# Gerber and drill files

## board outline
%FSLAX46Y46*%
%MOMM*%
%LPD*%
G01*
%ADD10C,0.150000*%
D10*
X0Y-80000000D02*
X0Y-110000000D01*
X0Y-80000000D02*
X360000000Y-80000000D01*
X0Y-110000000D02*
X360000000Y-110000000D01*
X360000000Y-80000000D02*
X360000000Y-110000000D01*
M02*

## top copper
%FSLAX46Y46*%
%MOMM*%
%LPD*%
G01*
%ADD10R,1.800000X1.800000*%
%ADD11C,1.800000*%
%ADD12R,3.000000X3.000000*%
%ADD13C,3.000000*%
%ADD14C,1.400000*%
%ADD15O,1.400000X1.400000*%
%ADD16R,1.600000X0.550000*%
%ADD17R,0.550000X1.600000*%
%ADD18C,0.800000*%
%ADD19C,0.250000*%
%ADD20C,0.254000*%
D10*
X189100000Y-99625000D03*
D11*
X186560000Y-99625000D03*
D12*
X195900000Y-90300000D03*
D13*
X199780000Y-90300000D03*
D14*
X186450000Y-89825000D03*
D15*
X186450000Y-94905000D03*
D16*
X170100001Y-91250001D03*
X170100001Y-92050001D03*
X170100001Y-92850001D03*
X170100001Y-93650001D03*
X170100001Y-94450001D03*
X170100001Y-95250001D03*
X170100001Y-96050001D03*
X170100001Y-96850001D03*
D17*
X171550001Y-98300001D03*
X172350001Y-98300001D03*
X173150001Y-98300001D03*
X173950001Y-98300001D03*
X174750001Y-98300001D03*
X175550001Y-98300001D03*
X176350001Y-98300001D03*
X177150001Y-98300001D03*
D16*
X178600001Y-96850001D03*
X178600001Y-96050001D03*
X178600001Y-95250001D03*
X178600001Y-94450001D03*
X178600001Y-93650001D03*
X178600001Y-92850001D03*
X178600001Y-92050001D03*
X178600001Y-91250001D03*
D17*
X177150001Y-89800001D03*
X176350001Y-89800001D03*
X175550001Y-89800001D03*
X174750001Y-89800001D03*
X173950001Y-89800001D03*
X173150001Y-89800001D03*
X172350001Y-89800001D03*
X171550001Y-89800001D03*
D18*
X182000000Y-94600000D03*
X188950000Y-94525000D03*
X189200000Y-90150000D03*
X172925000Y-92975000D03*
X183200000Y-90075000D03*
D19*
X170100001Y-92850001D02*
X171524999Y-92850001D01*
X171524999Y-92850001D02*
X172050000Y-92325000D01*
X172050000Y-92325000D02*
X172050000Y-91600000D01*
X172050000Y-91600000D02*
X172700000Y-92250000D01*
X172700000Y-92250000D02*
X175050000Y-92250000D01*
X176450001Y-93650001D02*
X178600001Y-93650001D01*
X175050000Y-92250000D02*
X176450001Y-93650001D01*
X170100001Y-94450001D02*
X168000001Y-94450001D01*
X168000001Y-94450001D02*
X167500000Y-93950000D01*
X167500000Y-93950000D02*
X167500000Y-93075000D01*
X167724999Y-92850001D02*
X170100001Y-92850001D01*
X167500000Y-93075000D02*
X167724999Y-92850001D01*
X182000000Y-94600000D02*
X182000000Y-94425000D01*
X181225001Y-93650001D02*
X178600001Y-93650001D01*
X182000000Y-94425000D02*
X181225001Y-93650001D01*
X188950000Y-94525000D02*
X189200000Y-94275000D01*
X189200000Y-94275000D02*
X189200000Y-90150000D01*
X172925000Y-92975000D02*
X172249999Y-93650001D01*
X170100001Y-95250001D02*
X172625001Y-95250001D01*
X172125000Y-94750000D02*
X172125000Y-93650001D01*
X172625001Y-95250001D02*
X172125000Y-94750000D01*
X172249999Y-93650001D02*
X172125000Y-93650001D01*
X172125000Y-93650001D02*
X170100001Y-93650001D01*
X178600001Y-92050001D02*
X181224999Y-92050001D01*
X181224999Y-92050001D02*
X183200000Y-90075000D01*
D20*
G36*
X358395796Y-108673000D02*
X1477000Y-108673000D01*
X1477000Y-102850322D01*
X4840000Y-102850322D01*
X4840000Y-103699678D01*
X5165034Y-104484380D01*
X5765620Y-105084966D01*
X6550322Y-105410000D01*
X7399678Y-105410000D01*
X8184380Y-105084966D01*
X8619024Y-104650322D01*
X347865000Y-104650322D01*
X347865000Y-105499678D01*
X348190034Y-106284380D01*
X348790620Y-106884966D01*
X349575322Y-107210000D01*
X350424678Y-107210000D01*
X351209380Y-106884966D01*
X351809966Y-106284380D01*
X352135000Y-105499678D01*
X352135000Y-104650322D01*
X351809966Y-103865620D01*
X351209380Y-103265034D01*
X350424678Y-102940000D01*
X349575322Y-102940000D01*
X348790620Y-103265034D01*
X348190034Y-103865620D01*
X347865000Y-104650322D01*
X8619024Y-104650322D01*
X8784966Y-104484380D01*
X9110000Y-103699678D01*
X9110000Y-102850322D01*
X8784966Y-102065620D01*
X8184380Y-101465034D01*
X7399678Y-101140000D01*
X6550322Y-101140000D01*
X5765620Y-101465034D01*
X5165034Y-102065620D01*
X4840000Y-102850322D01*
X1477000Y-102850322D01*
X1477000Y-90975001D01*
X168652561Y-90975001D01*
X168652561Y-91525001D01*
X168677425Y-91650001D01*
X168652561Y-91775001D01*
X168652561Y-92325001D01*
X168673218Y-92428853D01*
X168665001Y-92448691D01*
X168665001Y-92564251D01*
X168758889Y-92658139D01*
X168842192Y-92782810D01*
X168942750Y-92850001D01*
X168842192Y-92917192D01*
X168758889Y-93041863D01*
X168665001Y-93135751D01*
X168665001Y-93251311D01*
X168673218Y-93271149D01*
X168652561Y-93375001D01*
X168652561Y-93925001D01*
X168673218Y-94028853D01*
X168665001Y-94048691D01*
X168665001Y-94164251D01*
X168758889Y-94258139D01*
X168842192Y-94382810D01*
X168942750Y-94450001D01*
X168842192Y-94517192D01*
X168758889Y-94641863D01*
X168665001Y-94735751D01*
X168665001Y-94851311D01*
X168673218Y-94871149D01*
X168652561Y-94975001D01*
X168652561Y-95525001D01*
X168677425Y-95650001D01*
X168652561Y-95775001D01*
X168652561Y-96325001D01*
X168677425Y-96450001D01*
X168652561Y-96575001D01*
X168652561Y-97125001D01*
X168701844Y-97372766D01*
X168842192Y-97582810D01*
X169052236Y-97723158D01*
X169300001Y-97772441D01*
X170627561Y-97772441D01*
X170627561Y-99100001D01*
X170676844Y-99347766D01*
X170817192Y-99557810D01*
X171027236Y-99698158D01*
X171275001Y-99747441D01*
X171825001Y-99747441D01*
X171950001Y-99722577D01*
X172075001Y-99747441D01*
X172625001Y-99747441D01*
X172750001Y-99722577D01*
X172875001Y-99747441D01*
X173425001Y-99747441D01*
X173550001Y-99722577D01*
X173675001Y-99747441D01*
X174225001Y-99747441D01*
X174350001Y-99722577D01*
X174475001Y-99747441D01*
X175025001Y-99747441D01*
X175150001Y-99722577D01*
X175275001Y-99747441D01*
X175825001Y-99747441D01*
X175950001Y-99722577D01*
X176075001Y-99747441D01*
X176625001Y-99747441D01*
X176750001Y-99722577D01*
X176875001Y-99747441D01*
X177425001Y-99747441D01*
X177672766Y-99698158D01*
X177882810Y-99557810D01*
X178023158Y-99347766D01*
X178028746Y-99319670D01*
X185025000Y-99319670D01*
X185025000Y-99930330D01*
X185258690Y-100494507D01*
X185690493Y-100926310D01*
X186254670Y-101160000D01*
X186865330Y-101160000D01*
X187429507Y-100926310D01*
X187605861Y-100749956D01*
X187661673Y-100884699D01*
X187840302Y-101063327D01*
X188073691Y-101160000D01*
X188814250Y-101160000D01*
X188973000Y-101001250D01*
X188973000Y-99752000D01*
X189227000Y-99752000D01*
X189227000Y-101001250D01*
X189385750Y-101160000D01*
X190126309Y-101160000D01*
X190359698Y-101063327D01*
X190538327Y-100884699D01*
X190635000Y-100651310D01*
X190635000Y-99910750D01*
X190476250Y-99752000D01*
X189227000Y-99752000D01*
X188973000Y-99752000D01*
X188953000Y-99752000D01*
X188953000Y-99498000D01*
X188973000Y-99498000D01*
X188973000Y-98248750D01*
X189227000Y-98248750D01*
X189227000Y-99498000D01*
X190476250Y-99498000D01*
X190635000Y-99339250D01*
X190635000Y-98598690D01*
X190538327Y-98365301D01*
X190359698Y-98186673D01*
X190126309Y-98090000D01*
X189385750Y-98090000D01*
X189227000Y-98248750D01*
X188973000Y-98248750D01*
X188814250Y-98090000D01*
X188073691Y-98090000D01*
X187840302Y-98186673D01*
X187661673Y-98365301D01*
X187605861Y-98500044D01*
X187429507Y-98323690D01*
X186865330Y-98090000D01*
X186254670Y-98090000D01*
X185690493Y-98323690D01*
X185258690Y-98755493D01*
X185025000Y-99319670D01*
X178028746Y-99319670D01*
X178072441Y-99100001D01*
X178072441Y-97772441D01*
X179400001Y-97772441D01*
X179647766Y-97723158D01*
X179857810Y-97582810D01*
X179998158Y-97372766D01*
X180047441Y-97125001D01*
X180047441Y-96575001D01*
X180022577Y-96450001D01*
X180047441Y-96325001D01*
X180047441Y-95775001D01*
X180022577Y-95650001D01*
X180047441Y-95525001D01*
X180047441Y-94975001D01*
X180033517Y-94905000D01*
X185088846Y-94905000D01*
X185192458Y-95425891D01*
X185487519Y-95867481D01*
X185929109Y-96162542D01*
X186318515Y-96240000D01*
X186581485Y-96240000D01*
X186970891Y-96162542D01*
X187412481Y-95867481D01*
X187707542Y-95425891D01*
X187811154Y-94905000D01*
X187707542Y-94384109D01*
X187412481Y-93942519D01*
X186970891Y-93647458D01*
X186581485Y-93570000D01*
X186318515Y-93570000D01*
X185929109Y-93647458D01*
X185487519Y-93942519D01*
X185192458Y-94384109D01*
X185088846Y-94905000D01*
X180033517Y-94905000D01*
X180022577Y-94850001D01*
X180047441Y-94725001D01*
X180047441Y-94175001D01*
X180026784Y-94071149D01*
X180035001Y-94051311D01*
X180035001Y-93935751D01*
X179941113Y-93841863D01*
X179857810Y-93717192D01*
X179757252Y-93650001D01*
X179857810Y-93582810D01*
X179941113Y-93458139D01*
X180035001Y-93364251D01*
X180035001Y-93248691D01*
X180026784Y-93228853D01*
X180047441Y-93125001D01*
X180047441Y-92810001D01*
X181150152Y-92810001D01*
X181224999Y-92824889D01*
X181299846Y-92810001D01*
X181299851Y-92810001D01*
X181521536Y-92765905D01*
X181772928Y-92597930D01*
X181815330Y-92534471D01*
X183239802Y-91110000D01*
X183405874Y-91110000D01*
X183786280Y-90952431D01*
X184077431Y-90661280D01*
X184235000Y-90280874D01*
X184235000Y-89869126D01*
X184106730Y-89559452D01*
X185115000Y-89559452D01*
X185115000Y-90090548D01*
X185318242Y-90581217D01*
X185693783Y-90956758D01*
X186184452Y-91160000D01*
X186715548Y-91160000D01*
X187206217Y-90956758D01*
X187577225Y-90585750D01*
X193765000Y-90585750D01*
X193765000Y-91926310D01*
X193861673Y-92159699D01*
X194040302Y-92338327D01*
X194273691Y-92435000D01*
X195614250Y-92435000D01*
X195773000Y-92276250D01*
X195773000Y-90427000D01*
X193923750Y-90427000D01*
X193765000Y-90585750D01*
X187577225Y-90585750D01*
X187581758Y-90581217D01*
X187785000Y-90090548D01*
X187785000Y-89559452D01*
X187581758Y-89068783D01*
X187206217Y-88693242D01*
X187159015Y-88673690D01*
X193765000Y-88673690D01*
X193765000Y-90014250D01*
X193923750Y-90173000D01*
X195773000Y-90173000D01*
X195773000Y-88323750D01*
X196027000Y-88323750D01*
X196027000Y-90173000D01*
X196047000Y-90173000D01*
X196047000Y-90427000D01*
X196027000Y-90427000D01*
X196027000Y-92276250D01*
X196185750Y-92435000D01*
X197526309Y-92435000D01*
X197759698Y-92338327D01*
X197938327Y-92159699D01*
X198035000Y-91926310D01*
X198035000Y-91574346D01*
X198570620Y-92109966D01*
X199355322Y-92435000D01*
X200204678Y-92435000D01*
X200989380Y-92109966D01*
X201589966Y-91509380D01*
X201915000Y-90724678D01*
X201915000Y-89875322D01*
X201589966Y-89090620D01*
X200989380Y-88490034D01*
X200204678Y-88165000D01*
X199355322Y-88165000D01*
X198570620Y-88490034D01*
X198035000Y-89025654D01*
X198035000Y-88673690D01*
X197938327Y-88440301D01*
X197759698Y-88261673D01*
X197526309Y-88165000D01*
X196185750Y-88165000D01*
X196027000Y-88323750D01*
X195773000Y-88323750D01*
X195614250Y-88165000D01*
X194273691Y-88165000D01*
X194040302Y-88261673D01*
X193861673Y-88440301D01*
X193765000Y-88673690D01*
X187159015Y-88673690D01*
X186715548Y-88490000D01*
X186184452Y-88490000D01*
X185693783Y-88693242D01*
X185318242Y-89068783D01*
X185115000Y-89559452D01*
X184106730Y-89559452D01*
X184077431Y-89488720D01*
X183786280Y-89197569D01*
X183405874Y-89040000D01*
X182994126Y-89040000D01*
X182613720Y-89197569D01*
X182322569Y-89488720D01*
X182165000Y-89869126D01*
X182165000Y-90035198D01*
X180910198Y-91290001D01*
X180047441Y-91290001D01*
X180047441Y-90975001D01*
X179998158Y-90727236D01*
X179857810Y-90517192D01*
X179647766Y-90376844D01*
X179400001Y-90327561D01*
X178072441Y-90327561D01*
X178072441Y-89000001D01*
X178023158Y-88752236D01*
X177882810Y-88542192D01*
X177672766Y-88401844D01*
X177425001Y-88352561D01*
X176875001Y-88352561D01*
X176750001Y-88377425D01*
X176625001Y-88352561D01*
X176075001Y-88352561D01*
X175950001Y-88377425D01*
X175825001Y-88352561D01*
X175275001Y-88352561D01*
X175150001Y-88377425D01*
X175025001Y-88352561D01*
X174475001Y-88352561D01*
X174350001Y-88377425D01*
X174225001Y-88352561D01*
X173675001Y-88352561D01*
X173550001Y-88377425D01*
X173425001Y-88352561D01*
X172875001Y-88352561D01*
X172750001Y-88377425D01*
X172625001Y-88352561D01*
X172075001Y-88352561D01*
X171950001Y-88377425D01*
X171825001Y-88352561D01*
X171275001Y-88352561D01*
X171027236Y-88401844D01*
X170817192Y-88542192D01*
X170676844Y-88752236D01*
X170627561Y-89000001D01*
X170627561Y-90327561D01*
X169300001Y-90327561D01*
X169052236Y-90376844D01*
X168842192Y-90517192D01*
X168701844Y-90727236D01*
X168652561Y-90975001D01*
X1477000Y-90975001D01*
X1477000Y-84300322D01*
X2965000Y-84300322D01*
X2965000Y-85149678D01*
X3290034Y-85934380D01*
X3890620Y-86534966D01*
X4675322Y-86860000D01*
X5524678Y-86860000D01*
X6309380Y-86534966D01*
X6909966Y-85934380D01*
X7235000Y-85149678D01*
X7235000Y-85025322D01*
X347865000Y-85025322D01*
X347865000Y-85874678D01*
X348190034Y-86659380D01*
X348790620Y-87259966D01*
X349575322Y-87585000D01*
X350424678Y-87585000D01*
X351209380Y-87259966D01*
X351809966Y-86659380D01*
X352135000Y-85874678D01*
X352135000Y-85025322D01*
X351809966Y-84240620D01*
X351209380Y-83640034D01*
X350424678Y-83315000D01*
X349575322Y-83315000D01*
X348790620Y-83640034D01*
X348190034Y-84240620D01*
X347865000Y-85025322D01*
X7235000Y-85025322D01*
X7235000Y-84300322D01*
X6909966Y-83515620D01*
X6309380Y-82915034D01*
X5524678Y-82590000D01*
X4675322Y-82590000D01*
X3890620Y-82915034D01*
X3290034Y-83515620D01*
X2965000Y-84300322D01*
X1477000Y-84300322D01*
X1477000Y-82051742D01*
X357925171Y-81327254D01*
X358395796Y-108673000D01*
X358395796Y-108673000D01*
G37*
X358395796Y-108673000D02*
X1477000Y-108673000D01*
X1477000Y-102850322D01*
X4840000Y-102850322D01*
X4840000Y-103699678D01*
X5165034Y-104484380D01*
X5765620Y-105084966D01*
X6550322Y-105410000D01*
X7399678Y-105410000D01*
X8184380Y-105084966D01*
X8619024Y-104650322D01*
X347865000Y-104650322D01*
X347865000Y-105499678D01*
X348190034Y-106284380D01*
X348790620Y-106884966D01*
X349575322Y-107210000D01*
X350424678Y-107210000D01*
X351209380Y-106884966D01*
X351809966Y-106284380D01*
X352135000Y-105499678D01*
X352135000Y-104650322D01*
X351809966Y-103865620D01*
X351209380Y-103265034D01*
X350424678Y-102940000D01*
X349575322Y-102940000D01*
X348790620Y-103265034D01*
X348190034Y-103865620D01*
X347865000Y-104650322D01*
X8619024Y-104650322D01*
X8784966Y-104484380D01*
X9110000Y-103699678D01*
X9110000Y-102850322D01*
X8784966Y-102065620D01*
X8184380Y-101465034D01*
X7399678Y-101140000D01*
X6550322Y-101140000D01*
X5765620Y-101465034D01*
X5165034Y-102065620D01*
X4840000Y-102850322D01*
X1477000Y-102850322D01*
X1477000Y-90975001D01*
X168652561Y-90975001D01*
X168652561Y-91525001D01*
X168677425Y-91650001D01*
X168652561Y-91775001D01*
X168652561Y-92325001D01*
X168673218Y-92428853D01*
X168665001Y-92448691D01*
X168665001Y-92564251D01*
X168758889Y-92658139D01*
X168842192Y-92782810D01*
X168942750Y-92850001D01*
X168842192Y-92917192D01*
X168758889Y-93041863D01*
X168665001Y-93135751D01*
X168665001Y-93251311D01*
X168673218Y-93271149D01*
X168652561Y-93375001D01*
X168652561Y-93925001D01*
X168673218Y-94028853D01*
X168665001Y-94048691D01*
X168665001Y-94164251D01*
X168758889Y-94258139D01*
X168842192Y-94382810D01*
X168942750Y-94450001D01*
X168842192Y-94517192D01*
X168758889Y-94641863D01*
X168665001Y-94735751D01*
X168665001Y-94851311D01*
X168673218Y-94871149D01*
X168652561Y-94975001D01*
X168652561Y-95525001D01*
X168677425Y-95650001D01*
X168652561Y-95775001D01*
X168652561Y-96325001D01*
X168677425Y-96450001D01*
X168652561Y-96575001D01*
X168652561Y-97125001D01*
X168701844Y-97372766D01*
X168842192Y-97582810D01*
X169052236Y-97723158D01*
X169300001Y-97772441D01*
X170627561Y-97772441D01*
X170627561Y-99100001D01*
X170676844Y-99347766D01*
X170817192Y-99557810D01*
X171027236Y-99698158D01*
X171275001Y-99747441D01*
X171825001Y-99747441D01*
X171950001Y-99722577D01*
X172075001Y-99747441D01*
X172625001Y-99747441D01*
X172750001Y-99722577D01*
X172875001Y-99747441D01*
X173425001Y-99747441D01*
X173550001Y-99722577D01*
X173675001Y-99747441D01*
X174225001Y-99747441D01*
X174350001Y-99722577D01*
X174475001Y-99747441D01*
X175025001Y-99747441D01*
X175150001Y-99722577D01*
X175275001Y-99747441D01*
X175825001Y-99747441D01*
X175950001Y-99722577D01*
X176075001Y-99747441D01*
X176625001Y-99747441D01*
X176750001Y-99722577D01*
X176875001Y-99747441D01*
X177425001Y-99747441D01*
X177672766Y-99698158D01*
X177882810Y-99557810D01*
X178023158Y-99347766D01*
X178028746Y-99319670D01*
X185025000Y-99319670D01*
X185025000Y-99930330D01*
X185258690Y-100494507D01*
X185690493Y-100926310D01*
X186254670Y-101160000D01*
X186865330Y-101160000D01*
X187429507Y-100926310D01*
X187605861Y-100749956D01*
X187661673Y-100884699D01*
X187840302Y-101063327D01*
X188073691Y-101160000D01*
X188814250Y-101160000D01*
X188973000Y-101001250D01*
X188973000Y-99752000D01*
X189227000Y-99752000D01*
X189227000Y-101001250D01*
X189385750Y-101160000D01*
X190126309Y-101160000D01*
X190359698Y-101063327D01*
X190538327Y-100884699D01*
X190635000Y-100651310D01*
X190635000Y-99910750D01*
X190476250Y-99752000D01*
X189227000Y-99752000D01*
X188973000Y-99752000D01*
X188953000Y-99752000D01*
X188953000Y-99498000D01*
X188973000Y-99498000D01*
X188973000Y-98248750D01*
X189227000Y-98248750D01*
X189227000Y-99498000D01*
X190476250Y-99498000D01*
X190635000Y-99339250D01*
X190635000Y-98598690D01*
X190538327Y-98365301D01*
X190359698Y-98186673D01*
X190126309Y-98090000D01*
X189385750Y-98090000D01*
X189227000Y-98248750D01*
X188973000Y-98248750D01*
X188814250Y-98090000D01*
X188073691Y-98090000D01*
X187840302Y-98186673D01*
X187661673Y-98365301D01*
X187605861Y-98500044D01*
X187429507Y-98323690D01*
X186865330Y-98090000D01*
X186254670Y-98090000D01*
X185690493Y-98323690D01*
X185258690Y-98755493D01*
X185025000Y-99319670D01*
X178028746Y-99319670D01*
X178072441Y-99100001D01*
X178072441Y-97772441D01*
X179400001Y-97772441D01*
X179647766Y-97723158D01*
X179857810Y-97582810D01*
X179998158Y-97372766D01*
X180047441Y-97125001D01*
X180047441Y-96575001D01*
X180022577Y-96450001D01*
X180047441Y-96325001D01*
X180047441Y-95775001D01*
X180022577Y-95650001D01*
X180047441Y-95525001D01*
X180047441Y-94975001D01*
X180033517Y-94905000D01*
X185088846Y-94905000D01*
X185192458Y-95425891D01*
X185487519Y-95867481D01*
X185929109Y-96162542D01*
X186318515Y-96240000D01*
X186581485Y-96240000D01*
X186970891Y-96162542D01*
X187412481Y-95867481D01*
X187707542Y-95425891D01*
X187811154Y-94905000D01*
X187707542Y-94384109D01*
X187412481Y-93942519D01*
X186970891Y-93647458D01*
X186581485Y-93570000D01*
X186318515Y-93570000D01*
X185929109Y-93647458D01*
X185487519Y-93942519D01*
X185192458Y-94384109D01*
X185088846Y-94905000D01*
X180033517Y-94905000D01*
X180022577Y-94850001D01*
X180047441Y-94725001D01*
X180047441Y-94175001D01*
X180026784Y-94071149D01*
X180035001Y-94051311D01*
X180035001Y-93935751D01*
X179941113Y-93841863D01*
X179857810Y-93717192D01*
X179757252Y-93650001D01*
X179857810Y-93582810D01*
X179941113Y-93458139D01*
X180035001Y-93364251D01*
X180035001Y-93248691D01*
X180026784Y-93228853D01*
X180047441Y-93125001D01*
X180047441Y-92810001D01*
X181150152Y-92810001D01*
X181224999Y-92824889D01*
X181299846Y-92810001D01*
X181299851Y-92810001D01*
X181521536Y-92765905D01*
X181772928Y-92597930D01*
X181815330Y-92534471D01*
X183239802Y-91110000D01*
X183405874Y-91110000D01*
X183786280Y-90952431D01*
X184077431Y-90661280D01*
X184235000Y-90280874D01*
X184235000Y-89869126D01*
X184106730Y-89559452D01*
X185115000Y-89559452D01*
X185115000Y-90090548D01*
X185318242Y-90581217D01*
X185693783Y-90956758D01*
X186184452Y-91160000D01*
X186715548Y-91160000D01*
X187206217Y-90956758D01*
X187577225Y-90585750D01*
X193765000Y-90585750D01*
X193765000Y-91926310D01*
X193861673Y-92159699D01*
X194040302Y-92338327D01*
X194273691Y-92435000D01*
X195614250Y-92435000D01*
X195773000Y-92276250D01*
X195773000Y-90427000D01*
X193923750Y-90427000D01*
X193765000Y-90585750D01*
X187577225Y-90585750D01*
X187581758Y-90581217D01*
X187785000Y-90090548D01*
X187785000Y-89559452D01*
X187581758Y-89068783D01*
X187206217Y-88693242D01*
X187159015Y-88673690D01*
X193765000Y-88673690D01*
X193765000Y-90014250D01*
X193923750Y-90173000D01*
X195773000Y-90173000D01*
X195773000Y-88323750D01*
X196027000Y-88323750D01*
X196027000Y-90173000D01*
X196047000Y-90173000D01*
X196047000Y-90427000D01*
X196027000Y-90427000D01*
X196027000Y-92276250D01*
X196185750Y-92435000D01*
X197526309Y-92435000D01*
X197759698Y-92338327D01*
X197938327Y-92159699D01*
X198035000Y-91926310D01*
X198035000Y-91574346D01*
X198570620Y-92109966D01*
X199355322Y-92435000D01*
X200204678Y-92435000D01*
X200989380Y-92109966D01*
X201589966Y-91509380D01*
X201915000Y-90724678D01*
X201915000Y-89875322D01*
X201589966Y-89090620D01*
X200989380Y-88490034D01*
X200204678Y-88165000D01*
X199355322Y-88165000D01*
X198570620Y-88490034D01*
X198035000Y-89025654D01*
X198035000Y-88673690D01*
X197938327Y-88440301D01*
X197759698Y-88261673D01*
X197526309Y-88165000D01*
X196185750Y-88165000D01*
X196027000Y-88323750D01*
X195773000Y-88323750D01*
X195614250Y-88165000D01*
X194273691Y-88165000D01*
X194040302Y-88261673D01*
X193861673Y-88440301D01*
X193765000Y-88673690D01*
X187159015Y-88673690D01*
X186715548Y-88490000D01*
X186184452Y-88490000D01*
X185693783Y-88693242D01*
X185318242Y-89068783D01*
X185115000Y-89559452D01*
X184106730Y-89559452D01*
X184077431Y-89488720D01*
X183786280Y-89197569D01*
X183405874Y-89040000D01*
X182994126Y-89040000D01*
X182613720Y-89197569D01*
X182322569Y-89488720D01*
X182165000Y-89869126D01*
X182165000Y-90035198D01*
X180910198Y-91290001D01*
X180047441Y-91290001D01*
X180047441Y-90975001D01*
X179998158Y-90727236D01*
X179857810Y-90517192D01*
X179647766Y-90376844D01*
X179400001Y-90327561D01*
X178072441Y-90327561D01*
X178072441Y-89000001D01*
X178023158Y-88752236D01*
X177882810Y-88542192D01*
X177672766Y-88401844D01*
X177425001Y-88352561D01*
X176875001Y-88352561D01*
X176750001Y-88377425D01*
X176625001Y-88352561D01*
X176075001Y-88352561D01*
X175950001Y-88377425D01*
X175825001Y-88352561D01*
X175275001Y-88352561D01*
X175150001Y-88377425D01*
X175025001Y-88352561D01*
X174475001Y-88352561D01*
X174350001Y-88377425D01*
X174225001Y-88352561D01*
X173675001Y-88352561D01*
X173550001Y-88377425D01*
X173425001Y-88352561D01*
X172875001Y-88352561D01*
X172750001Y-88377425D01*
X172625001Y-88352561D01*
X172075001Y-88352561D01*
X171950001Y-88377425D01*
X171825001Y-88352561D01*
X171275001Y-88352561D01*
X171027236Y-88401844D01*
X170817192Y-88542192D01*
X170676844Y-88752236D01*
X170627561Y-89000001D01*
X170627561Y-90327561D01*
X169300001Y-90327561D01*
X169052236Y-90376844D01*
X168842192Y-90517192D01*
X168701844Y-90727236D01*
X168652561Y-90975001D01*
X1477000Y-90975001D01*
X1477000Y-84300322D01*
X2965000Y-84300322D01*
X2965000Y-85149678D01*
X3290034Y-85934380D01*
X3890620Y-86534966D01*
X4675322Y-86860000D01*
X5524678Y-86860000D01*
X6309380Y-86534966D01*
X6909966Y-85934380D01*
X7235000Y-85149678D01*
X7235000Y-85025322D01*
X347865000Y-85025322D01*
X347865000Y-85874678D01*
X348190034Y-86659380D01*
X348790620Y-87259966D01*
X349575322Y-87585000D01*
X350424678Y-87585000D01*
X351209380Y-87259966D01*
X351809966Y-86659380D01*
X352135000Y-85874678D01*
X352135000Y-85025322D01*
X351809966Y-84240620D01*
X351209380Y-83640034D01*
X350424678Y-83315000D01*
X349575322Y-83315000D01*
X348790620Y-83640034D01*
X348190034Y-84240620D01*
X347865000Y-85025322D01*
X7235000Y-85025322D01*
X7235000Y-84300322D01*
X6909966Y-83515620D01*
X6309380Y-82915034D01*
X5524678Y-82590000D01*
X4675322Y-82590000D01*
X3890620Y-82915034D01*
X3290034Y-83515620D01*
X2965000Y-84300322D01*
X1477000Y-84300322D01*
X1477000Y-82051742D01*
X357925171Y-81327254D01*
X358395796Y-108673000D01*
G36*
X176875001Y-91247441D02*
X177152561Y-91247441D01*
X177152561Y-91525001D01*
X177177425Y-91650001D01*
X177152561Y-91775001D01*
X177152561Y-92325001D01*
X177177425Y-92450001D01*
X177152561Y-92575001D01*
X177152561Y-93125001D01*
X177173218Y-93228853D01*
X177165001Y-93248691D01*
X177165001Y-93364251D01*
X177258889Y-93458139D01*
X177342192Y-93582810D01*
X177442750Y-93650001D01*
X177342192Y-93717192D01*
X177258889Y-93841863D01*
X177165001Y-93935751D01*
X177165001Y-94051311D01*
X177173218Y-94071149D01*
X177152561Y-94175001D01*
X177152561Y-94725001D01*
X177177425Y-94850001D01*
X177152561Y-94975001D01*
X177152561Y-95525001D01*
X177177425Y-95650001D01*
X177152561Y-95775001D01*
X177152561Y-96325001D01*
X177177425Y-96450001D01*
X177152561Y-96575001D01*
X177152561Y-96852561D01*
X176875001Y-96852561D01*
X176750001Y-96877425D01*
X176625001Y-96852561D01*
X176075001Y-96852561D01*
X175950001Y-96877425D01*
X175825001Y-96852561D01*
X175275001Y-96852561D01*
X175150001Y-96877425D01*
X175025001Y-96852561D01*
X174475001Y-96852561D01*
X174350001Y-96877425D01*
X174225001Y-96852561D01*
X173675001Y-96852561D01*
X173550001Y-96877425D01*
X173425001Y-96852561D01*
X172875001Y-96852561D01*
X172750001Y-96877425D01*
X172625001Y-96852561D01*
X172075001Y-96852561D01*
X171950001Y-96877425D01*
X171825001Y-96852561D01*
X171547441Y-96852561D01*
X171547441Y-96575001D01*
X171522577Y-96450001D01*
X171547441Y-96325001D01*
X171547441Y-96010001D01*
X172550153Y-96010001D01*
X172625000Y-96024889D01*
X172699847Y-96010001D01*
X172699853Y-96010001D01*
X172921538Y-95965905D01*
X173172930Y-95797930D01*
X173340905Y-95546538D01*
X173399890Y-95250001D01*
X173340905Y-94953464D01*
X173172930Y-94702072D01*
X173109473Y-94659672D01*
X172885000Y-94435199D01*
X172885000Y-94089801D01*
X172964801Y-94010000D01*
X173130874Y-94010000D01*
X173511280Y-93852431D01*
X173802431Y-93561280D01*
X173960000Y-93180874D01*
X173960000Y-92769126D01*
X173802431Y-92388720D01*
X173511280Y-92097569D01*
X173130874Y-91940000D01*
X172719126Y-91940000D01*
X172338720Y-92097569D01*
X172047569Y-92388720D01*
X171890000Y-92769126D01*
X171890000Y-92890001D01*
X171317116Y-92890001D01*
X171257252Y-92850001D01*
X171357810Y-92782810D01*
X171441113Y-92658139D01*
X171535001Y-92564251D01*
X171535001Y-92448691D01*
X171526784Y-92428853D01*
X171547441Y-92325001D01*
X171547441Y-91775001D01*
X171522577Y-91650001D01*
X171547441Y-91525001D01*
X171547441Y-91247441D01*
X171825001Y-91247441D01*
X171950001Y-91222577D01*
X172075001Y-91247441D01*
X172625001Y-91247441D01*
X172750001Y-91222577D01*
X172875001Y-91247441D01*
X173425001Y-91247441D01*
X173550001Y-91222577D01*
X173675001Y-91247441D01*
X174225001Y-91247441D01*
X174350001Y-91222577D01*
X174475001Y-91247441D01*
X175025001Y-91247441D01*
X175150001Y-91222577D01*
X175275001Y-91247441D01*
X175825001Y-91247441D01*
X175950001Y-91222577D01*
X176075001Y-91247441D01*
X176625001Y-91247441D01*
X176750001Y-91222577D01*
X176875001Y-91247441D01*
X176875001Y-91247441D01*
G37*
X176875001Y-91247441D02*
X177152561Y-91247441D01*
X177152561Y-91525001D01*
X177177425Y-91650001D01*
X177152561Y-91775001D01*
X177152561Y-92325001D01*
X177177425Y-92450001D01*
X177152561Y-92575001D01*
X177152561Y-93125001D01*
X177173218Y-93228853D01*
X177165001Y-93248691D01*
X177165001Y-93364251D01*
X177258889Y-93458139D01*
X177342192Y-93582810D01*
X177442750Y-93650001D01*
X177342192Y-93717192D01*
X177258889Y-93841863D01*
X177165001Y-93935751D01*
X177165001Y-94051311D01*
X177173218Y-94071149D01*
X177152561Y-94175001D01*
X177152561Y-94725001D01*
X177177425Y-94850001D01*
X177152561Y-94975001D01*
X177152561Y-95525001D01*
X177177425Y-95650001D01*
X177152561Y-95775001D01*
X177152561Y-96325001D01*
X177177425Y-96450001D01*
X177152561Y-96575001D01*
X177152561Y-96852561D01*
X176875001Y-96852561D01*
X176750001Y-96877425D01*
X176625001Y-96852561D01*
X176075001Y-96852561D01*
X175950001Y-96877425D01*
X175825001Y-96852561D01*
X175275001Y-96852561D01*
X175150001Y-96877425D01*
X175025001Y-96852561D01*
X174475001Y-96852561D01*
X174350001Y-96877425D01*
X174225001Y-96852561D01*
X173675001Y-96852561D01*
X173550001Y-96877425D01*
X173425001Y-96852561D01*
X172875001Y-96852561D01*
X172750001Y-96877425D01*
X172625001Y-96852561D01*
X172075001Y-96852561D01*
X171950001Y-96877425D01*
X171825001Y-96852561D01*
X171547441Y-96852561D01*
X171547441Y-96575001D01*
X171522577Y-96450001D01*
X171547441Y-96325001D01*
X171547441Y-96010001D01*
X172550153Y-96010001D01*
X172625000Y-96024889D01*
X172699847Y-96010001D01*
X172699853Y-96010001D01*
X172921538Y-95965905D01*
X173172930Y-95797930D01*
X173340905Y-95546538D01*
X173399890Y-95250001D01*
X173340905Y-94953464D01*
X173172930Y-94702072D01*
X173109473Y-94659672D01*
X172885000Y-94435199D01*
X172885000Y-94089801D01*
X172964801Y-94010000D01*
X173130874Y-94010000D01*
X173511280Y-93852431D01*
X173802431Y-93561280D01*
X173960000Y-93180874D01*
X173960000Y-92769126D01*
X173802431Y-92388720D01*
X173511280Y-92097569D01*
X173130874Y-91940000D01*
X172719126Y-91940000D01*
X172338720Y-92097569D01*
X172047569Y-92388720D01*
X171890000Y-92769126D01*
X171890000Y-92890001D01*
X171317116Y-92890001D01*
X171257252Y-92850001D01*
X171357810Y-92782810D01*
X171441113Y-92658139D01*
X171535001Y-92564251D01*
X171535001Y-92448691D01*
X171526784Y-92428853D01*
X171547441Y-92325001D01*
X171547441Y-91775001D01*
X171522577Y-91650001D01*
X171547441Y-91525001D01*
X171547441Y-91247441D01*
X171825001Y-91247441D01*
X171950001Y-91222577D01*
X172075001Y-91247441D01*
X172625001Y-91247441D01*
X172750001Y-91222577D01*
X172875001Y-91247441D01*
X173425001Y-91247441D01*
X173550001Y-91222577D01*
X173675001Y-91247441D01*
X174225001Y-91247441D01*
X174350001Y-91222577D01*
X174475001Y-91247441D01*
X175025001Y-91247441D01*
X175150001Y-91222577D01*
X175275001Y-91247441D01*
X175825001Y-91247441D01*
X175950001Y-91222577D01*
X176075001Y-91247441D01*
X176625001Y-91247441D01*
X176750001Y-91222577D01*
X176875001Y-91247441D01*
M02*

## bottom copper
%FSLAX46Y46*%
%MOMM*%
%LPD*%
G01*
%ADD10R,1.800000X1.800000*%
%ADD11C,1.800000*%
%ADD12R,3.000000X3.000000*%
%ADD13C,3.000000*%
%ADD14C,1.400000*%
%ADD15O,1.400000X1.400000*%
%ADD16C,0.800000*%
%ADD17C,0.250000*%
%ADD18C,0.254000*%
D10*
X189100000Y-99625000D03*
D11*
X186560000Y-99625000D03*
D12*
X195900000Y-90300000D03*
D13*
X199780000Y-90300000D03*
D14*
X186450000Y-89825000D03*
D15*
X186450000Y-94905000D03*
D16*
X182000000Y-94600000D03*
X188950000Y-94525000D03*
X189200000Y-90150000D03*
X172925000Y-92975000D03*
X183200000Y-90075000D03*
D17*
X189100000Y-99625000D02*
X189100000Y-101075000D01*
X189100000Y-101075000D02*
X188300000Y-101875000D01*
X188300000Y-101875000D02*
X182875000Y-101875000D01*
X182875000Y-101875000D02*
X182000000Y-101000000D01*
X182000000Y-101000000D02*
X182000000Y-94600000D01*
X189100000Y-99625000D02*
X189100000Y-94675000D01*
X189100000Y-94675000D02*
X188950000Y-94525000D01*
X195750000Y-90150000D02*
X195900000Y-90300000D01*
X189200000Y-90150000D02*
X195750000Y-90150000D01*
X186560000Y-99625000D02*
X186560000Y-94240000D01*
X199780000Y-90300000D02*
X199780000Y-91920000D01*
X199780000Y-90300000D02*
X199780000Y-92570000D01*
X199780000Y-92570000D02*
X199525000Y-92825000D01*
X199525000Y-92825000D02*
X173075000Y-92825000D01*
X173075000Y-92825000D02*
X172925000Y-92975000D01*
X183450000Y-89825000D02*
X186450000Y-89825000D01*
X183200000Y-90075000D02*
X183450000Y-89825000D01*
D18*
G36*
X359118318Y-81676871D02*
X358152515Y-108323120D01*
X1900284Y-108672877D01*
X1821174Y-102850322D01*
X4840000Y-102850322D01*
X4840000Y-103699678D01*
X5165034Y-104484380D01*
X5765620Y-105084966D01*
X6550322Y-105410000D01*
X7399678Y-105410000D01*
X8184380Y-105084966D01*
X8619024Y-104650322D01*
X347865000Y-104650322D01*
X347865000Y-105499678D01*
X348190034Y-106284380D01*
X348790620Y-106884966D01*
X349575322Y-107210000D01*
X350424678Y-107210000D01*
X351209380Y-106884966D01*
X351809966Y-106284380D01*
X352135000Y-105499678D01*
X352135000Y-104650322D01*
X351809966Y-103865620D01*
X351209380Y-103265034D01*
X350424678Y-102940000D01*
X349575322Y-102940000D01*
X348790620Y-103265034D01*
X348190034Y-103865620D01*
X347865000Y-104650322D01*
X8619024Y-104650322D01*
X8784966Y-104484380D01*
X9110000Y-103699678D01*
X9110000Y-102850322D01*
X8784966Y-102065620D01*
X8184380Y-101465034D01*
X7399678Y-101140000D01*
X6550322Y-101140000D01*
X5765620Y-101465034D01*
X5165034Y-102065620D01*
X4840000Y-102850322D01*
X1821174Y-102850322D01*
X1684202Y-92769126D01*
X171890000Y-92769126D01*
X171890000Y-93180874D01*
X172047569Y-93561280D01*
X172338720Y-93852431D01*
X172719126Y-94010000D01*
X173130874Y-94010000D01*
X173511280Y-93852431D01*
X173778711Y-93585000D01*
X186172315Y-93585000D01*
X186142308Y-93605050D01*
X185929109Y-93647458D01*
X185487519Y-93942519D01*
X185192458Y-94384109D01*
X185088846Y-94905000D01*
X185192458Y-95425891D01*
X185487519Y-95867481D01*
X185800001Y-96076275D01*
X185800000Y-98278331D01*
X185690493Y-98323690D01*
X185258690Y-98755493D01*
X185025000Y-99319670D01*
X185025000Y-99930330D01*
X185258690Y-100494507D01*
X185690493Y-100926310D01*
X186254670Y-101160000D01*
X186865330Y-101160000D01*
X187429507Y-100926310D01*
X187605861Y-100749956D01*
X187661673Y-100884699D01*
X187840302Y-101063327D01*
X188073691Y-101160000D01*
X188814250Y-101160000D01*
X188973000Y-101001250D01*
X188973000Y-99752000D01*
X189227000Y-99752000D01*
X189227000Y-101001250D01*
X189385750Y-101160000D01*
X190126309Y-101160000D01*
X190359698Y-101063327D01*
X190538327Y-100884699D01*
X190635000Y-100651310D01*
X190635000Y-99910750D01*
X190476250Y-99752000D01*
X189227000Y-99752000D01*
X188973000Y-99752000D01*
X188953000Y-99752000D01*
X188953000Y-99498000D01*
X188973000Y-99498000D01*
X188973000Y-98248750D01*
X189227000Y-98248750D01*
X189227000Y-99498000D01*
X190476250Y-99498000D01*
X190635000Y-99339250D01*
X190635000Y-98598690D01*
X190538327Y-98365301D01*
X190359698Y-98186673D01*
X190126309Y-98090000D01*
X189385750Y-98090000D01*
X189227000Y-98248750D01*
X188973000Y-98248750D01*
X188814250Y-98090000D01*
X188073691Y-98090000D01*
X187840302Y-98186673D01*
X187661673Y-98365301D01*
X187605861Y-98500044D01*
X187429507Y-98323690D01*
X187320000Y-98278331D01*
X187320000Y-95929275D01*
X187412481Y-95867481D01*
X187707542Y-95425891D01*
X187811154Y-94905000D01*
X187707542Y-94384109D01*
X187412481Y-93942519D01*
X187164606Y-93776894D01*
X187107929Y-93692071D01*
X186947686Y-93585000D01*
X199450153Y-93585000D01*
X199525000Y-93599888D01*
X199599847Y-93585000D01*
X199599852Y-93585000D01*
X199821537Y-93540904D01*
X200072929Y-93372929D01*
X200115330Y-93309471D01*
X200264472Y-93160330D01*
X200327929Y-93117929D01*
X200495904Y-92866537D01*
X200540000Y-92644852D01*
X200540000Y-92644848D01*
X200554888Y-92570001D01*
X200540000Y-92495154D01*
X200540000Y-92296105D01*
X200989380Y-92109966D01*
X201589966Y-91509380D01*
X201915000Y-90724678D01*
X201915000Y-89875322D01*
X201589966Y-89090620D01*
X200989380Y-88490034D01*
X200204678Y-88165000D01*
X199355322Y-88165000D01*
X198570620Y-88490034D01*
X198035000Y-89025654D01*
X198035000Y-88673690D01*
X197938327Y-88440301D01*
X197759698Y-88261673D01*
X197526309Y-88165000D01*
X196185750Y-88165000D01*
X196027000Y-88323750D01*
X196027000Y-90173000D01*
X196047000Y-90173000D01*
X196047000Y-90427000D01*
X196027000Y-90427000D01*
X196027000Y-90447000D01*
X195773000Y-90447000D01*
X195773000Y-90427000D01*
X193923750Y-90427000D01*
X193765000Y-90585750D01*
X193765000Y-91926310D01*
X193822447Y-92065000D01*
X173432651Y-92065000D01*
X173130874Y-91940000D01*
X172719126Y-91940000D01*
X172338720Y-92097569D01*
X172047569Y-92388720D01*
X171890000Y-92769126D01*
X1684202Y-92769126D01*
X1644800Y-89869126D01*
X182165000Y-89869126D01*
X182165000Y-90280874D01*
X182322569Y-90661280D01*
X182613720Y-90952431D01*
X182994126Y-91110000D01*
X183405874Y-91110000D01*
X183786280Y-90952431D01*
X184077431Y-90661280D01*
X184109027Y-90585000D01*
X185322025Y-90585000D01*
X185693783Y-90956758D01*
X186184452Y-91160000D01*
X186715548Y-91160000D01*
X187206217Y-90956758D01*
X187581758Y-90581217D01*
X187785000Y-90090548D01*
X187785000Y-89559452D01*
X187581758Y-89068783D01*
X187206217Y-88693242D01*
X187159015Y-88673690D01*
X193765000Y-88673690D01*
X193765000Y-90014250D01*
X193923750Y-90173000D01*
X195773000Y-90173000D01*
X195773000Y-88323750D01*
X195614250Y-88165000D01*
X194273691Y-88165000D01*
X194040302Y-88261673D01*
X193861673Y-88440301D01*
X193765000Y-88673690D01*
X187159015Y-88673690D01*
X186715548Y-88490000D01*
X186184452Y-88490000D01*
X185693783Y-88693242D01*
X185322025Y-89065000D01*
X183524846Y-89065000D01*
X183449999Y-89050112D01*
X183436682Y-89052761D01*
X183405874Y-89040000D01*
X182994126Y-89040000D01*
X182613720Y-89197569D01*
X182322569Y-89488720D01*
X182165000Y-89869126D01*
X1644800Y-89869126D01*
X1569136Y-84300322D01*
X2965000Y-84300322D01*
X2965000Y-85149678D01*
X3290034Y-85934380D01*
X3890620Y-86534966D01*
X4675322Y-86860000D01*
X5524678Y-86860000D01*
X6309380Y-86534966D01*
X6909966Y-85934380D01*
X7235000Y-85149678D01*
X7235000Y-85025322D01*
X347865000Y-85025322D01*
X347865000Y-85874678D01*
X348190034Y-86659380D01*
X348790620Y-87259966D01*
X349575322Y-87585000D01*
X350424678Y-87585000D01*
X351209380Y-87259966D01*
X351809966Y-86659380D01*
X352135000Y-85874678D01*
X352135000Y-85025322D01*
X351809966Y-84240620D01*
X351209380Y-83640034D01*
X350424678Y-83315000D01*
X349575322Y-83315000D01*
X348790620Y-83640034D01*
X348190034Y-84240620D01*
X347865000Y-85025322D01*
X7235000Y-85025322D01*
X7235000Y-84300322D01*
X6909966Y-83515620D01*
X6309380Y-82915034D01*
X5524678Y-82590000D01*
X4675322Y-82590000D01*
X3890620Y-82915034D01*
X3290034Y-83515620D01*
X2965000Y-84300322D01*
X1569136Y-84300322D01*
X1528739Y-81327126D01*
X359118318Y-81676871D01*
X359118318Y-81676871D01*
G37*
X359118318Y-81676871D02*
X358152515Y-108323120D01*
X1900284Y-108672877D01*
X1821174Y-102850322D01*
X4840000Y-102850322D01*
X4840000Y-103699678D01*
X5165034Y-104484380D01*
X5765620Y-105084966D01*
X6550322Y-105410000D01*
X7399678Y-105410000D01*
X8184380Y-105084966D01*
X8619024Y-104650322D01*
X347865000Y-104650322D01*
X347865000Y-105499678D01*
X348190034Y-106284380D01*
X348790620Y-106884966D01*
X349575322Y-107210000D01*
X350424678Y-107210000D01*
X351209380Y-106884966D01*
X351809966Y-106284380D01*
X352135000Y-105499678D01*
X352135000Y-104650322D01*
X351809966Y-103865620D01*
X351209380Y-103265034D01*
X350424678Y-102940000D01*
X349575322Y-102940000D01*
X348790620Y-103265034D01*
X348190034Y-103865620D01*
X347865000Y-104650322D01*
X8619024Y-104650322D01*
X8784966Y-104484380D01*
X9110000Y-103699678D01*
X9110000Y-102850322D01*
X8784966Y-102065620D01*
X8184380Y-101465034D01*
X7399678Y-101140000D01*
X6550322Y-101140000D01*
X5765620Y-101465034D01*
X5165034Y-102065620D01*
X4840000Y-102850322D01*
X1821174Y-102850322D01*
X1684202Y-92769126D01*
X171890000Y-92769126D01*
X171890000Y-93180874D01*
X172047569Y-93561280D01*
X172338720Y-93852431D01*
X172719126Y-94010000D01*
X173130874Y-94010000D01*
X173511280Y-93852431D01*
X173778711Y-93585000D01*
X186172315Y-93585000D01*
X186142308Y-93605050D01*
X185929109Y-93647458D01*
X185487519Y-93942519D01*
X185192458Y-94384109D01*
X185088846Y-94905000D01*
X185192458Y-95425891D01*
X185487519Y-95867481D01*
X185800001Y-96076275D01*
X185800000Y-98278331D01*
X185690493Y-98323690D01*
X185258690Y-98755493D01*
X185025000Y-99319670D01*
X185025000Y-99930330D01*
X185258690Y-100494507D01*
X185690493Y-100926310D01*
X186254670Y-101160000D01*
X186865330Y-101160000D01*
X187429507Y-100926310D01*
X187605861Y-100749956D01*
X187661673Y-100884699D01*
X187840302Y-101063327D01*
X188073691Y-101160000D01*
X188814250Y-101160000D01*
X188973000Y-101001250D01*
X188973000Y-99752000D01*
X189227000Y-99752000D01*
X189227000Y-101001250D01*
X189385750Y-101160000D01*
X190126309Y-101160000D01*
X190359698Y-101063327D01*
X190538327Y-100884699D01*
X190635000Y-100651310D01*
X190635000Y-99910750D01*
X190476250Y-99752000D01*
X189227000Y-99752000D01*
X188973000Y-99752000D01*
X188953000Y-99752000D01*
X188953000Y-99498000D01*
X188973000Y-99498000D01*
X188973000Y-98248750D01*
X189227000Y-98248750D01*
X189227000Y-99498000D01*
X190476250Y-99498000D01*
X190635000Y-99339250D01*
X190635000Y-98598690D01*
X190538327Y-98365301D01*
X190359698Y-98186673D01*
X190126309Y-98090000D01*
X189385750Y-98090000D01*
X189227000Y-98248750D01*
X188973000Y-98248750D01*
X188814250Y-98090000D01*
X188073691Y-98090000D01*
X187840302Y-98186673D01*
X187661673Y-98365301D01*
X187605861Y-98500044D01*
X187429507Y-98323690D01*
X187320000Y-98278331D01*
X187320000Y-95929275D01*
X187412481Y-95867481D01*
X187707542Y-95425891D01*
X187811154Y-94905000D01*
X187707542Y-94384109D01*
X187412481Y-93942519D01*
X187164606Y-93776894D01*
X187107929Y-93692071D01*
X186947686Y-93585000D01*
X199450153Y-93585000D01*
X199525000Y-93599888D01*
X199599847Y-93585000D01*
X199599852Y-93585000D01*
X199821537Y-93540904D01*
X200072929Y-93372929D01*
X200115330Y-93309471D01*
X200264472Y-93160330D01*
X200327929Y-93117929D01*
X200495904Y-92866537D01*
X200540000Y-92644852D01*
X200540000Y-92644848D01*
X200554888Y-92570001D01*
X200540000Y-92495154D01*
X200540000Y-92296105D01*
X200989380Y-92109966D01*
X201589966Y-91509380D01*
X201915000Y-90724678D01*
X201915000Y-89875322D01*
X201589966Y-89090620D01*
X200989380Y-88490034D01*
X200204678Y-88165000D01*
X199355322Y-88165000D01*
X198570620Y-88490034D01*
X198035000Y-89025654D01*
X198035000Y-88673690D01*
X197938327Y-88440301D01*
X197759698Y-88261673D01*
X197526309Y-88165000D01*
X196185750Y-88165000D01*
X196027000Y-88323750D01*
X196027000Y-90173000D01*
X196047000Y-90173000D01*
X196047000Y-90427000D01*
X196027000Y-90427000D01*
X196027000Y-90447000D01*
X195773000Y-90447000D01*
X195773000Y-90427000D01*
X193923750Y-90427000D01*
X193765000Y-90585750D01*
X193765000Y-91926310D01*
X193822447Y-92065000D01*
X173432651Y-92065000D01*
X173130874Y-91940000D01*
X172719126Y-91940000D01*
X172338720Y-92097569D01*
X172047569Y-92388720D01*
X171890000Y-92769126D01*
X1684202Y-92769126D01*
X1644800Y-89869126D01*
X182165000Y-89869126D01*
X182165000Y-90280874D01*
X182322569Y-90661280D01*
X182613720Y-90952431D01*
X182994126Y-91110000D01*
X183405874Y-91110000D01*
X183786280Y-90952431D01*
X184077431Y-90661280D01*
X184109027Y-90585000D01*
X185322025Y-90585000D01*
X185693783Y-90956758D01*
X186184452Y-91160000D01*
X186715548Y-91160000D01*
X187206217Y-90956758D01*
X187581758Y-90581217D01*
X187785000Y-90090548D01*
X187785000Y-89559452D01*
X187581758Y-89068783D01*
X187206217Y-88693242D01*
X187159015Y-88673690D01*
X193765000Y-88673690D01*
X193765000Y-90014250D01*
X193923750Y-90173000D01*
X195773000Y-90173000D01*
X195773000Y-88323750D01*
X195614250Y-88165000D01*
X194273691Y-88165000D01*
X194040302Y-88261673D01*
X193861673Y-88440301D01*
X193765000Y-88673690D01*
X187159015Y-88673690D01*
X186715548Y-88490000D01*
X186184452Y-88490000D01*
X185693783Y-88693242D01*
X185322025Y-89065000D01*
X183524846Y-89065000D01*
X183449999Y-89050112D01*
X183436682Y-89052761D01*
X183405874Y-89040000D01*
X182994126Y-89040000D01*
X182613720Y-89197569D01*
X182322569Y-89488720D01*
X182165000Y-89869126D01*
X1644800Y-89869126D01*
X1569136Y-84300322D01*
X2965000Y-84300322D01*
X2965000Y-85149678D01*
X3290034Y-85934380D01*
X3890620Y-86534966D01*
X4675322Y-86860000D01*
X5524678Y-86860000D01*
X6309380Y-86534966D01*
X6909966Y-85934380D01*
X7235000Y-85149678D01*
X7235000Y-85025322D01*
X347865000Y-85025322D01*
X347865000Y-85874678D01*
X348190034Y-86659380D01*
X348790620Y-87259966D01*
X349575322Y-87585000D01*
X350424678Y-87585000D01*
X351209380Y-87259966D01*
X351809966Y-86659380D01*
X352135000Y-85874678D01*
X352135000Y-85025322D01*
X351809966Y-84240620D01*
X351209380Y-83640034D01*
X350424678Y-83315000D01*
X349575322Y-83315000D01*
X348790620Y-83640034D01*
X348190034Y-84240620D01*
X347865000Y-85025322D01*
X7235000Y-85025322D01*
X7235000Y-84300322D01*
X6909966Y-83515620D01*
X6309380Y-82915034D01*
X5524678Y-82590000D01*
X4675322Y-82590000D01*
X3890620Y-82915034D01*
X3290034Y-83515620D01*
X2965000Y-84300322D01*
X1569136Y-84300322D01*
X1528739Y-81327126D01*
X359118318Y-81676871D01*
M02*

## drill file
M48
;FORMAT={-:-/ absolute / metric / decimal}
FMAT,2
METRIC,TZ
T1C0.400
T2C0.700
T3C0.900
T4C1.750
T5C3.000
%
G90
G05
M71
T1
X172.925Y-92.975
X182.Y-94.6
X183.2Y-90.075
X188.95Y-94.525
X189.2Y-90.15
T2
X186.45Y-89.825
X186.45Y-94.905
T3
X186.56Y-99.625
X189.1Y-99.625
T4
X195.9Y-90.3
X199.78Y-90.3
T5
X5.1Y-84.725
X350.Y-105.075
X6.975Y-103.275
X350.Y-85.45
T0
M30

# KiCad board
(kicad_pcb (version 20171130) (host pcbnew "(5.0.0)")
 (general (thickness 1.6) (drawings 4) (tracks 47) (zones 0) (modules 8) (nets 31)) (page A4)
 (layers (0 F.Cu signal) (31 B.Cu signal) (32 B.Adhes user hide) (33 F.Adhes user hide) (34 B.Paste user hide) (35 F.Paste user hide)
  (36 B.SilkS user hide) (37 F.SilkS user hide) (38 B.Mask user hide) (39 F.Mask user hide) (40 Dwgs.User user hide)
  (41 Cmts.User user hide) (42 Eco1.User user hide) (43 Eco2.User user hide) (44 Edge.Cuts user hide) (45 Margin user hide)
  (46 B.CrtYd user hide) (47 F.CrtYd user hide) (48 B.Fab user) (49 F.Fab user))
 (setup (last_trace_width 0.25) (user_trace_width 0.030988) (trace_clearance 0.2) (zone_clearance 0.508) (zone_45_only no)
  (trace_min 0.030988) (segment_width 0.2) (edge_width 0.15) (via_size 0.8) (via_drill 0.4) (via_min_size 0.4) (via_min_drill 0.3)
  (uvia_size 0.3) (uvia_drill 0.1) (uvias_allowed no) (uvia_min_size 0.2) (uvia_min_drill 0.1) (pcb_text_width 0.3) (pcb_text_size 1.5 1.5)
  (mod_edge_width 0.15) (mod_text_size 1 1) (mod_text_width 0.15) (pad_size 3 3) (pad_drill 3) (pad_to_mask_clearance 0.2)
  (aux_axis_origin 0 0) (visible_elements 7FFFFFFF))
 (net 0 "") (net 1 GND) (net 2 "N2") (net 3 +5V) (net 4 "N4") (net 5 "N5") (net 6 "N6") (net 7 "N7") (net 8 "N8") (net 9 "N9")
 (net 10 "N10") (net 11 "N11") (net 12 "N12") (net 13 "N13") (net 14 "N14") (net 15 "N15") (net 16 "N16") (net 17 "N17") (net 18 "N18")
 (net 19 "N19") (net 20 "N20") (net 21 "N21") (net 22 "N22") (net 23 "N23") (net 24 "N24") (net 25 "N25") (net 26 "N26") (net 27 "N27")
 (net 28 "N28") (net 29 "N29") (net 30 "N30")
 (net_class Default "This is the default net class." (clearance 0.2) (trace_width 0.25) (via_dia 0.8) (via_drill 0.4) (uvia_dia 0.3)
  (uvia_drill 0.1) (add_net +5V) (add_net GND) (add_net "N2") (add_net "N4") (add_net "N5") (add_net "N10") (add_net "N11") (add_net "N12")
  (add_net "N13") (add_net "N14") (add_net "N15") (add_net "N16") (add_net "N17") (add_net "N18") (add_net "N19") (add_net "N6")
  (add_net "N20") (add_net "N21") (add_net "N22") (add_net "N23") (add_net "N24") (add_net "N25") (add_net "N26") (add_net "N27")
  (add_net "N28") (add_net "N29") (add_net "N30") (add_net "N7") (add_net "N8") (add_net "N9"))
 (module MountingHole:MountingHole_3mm (layer F.Cu) (at 5.1 84.725)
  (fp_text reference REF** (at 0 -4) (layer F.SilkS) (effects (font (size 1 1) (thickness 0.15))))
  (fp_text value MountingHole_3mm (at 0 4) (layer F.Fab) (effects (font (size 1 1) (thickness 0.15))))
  (pad 1 np_thru_hole circle (at 0 0) (size 3 3) (drill 3) (layers *.Cu *.Mask)))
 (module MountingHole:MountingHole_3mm (layer F.Cu) (at 6.975 103.275)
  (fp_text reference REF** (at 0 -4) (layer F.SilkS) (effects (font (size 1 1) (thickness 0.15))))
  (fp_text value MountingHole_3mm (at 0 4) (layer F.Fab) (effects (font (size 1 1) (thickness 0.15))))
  (pad 1 np_thru_hole circle (at 0 0) (size 3 3) (drill 3) (layers *.Cu *.Mask)))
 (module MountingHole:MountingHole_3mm (layer F.Cu) (at 350 85.45 90)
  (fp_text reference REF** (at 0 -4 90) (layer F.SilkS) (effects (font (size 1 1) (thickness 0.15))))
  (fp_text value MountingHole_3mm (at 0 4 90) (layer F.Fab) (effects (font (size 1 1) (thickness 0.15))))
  (pad 1 np_thru_hole circle (at 0 0 90) (size 3 3) (drill 3) (layers *.Cu *.Mask)))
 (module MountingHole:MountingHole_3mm (layer F.Cu) (at 350 105.075)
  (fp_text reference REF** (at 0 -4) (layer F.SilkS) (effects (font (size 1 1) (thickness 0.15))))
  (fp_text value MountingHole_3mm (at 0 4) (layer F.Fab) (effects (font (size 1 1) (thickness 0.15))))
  (pad 1 np_thru_hole circle (at 0 0) (size 3 3) (drill 3) (layers *.Cu *.Mask)))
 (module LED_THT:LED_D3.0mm (layer F.Cu) (at 189.1 99.625 180)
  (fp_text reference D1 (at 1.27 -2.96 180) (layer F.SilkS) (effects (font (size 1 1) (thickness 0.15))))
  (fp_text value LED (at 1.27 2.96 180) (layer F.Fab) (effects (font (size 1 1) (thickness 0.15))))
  (pad 1 thru_hole rect (at 0 0 180) (size 1.8 1.8) (drill 0.9) (layers *.Cu *.Mask) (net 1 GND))
  (pad 2 thru_hole circle (at 2.54 0 180) (size 1.8 1.8) (drill 0.9) (layers *.Cu *.Mask) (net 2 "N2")))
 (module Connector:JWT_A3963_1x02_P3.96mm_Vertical (layer F.Cu) (at 195.9 90.3)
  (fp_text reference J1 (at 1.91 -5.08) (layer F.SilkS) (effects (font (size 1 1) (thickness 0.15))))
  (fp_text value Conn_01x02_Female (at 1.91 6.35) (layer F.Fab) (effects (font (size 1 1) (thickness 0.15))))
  (pad 1 thru_hole rect (at 0 0) (size 3 3) (drill 1.75) (layers *.Cu *.Mask) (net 1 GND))
  (pad 2 thru_hole circle (at 3.88 0) (size 3 3) (drill 1.75) (layers *.Cu *.Mask) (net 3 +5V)))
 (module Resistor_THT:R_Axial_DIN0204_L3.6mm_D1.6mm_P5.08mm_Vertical (layer F.Cu) (at 186.45 89.825 270)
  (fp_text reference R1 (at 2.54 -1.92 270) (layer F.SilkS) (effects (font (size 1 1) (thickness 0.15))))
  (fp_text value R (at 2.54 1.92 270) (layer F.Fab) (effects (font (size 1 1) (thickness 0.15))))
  (pad 1 thru_hole circle (at 0 0 270) (size 1.4 1.4) (drill 0.7) (layers *.Cu *.Mask) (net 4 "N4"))
  (pad 2 thru_hole oval (at 5.08 0 270) (size 1.4 1.4) (drill 0.7) (layers *.Cu *.Mask) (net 2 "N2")))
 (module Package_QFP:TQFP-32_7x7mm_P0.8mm (layer F.Cu) (at 174.350001 94.050001)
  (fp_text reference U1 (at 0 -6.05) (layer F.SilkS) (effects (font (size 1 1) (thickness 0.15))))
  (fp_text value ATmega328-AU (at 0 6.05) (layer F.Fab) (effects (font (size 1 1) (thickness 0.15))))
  (pad 1 smd rect (at -4.25 -2.8) (size 1.6 0.55) (layers F.Cu F.Paste F.Mask) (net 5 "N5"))
  (pad 2 smd rect (at -4.25 -2) (size 1.6 0.55) (layers F.Cu F.Paste F.Mask) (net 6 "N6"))
  (pad 3 smd rect (at -4.25 -1.2) (size 1.6 0.55) (layers F.Cu F.Paste F.Mask) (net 1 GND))
  (pad 4 smd rect (at -4.25 -0.4) (size 1.6 0.55) (layers F.Cu F.Paste F.Mask) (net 3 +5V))
  (pad 5 smd rect (at -4.25 0.4) (size 1.6 0.55) (layers F.Cu F.Paste F.Mask) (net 1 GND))
  (pad 6 smd rect (at -4.25 1.2) (size 1.6 0.55) (layers F.Cu F.Paste F.Mask) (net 3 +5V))
  (pad 7 smd rect (at -4.25 2) (size 1.6 0.55) (layers F.Cu F.Paste F.Mask) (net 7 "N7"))
  (pad 8 smd rect (at -4.25 2.8) (size 1.6 0.55) (layers F.Cu F.Paste F.Mask) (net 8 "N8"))
  (pad 9 smd rect (at -2.8 4.25 90) (size 1.6 0.55) (layers F.Cu F.Paste F.Mask) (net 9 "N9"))
  (pad 10 smd rect (at -2 4.25 90) (size 1.6 0.55) (layers F.Cu F.Paste F.Mask) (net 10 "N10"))
  (pad 11 smd rect (at -1.2 4.25 90) (size 1.6 0.55) (layers F.Cu F.Paste F.Mask) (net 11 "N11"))
  (pad 12 smd rect (at -0.4 4.25 90) (size 1.6 0.55) (layers F.Cu F.Paste F.Mask) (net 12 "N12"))
  (pad 13 smd rect (at 0.4 4.25 90) (size 1.6 0.55) (layers F.Cu F.Paste F.Mask) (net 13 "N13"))
  (pad 14 smd rect (at 1.2 4.25 90) (size 1.6 0.55) (layers F.Cu F.Paste F.Mask) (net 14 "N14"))
  (pad 15 smd rect (at 2 4.25 90) (size 1.6 0.55) (layers F.Cu F.Paste F.Mask) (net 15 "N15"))
  (pad 16 smd rect (at 2.8 4.25 90) (size 1.6 0.55) (layers F.Cu F.Paste F.Mask) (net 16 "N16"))
  (pad 17 smd rect (at 4.25 2.8) (size 1.6 0.55) (layers F.Cu F.Paste F.Mask) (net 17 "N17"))
  (pad 18 smd rect (at 4.25 2) (size 1.6 0.55) (layers F.Cu F.Paste F.Mask) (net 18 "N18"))
  (pad 19 smd rect (at 4.25 1.2) (size 1.6 0.55) (layers F.Cu F.Paste F.Mask) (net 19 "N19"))
  (pad 20 smd rect (at 4.25 0.4) (size 1.6 0.55) (layers F.Cu F.Paste F.Mask) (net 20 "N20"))
  (pad 21 smd rect (at 4.25 -0.4) (size 1.6 0.55) (layers F.Cu F.Paste F.Mask) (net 1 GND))
  (pad 22 smd rect (at 4.25 -1.2) (size 1.6 0.55) (layers F.Cu F.Paste F.Mask) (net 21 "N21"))
  (pad 23 smd rect (at 4.25 -2) (size 1.6 0.55) (layers F.Cu F.Paste F.Mask) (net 4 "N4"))
  (pad 24 smd rect (at 4.25 -2.8) (size 1.6 0.55) (layers F.Cu F.Paste F.Mask) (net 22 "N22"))
  (pad 25 smd rect (at 2.8 -4.25 90) (size 1.6 0.55) (layers F.Cu F.Paste F.Mask) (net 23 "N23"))
  (pad 26 smd rect (at 2 -4.25 90) (size 1.6 0.55) (layers F.Cu F.Paste F.Mask) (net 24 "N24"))
  (pad 27 smd rect (at 1.2 -4.25 90) (size 1.6 0.55) (layers F.Cu F.Paste F.Mask) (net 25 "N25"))
  (pad 28 smd rect (at 0.4 -4.25 90) (size 1.6 0.55) (layers F.Cu F.Paste F.Mask) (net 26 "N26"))
  (pad 29 smd rect (at -0.4 -4.25 90) (size 1.6 0.55) (layers F.Cu F.Paste F.Mask) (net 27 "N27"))
  (pad 30 smd rect (at -1.2 -4.25 90) (size 1.6 0.55) (layers F.Cu F.Paste F.Mask) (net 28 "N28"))
  (pad 31 smd rect (at -2 -4.25 90) (size 1.6 0.55) (layers F.Cu F.Paste F.Mask) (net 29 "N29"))
  (pad 32 smd rect (at -2.8 -4.25 90) (size 1.6 0.55) (layers F.Cu F.Paste F.Mask) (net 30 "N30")))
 (gr_line (start 0 80) (end 0 110) (layer Edge.Cuts) (width 0.15))
 (gr_line (start 0 80) (end 360 80) (layer Edge.Cuts) (width 0.15))
 (gr_line (start 0 110) (end 360 110) (layer Edge.Cuts) (width 0.15))
 (gr_line (start 360 80) (end 360 110) (layer Edge.Cuts) (width 0.15))
 (segment (start 170.100001 92.850001) (end 171.524999 92.850001) (width 0.25) (layer F.Cu) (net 1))
 (segment (start 171.524999 92.850001) (end 172.05 92.325) (width 0.25) (layer F.Cu) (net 1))
 (segment (start 172.05 92.325) (end 172.05 91.6) (width 0.25) (layer F.Cu) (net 1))
 (segment (start 172.05 91.6) (end 172.7 92.25) (width 0.25) (layer F.Cu) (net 1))
 (segment (start 172.7 92.25) (end 175.05 92.25) (width 0.25) (layer F.Cu) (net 1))
 (segment (start 176.450001 93.650001) (end 178.600001 93.650001) (width 0.25) (layer F.Cu) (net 1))
 (segment (start 175.05 92.25) (end 176.450001 93.650001) (width 0.25) (layer F.Cu) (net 1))
 (segment (start 170.100001 94.450001) (end 168.000001 94.450001) (width 0.25) (layer F.Cu) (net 1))
 (segment (start 168.000001 94.450001) (end 167.5 93.95) (width 0.25) (layer F.Cu) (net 1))
 (segment (start 167.5 93.95) (end 167.5 93.075) (width 0.25) (layer F.Cu) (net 1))
 (segment (start 167.724999 92.850001) (end 170.100001 92.850001) (width 0.25) (layer F.Cu) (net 1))
 (segment (start 167.5 93.075) (end 167.724999 92.850001) (width 0.25) (layer F.Cu) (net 1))
 (segment (start 189.1 99.625) (end 189.1 101.075) (width 0.25) (layer B.Cu) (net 1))
 (segment (start 189.1 101.075) (end 188.3 101.875) (width 0.25) (layer B.Cu) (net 1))
 (segment (start 188.3 101.875) (end 182.875 101.875) (width 0.25) (layer B.Cu) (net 1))
 (via (at 182 94.6) (size 0.8) (drill 0.4) (layers F.Cu B.Cu) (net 1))
 (segment (start 182.875 101.875) (end 182 101) (width 0.25) (layer B.Cu) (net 1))
 (segment (start 182 101) (end 182 94.6) (width 0.25) (layer B.Cu) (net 1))
 (segment (start 182 94.6) (end 182 94.425) (width 0.25) (layer F.Cu) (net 1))
 (segment (start 181.225001 93.650001) (end 178.600001 93.650001) (width 0.25) (layer F.Cu) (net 1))
 (segment (start 182 94.425) (end 181.225001 93.650001) (width 0.25) (layer F.Cu) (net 1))
 (via (at 188.95 94.525) (size 0.8) (drill 0.4) (layers F.Cu B.Cu) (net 1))
 (segment (start 189.1 99.625) (end 189.1 94.675) (width 0.25) (layer B.Cu) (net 1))
 (segment (start 189.1 94.675) (end 188.95 94.525) (width 0.25) (layer B.Cu) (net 1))
 (via (at 189.2 90.15) (size 0.8) (drill 0.4) (layers F.Cu B.Cu) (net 1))
 (segment (start 188.95 94.525) (end 189.2 94.275) (width 0.25) (layer F.Cu) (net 1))
 (segment (start 189.2 94.275) (end 189.2 90.15) (width 0.25) (layer F.Cu) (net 1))
 (segment (start 195.75 90.15) (end 195.9 90.3) (width 0.25) (layer B.Cu) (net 1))
 (segment (start 189.2 90.15) (end 195.75 90.15) (width 0.25) (layer B.Cu) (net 1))
 (segment (start 186.56 99.625) (end 186.56 94.24) (width 0.25) (layer B.Cu) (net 2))
 (segment (start 199.78 90.3) (end 199.78 91.92) (width 0.25) (layer B.Cu) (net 3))
 (segment (start 199.78 90.3) (end 199.78 92.57) (width 0.25) (layer B.Cu) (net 3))
 (segment (start 199.78 92.57) (end 199.525 92.825) (width 0.25) (layer B.Cu) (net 3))
 (via (at 172.925 92.975) (size 0.8) (drill 0.4) (layers F.Cu B.Cu) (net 3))
 (segment (start 199.525 92.825) (end 173.075 92.825) (width 0.25) (layer B.Cu) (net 3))
 (segment (start 173.075 92.825) (end 172.925 92.975) (width 0.25) (layer B.Cu) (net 3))
 (segment (start 172.925 92.975) (end 172.249999 93.650001) (width 0.25) (layer F.Cu) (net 3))
 (segment (start 170.100001 95.250001) (end 172.625001 95.250001) (width 0.25) (layer F.Cu) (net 3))
 (segment (start 172.125 94.75) (end 172.125 93.650001) (width 0.25) (layer F.Cu) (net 3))
 (segment (start 172.625001 95.250001) (end 172.125 94.75) (width 0.25) (layer F.Cu) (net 3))
 (segment (start 172.249999 93.650001) (end 172.125 93.650001) (width 0.25) (layer F.Cu) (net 3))
 (segment (start 172.125 93.650001) (end 170.100001 93.650001) (width 0.25) (layer F.Cu) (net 3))
 (via (at 183.2 90.075) (size 0.8) (drill 0.4) (layers F.Cu B.Cu) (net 4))
 (segment (start 178.600001 92.050001) (end 181.224999 92.050001) (width 0.25) (layer F.Cu) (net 4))
 (segment (start 181.224999 92.050001) (end 183.2 90.075) (width 0.25) (layer F.Cu) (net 4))
 (segment (start 183.45 89.825) (end 186.45 89.825) (width 0.25) (layer B.Cu) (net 4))
 (segment (start 183.2 90.075) (end 183.45 89.825) (width 0.25) (layer B.Cu) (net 4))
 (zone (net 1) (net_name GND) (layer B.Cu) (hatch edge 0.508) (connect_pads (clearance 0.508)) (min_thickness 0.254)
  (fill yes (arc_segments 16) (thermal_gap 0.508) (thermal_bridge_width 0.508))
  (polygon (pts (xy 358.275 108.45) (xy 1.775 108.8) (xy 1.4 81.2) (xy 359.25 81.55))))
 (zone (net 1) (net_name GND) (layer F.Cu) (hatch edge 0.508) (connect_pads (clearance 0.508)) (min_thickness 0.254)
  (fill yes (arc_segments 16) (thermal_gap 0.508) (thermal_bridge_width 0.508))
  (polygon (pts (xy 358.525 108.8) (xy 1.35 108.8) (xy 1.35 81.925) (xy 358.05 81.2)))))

